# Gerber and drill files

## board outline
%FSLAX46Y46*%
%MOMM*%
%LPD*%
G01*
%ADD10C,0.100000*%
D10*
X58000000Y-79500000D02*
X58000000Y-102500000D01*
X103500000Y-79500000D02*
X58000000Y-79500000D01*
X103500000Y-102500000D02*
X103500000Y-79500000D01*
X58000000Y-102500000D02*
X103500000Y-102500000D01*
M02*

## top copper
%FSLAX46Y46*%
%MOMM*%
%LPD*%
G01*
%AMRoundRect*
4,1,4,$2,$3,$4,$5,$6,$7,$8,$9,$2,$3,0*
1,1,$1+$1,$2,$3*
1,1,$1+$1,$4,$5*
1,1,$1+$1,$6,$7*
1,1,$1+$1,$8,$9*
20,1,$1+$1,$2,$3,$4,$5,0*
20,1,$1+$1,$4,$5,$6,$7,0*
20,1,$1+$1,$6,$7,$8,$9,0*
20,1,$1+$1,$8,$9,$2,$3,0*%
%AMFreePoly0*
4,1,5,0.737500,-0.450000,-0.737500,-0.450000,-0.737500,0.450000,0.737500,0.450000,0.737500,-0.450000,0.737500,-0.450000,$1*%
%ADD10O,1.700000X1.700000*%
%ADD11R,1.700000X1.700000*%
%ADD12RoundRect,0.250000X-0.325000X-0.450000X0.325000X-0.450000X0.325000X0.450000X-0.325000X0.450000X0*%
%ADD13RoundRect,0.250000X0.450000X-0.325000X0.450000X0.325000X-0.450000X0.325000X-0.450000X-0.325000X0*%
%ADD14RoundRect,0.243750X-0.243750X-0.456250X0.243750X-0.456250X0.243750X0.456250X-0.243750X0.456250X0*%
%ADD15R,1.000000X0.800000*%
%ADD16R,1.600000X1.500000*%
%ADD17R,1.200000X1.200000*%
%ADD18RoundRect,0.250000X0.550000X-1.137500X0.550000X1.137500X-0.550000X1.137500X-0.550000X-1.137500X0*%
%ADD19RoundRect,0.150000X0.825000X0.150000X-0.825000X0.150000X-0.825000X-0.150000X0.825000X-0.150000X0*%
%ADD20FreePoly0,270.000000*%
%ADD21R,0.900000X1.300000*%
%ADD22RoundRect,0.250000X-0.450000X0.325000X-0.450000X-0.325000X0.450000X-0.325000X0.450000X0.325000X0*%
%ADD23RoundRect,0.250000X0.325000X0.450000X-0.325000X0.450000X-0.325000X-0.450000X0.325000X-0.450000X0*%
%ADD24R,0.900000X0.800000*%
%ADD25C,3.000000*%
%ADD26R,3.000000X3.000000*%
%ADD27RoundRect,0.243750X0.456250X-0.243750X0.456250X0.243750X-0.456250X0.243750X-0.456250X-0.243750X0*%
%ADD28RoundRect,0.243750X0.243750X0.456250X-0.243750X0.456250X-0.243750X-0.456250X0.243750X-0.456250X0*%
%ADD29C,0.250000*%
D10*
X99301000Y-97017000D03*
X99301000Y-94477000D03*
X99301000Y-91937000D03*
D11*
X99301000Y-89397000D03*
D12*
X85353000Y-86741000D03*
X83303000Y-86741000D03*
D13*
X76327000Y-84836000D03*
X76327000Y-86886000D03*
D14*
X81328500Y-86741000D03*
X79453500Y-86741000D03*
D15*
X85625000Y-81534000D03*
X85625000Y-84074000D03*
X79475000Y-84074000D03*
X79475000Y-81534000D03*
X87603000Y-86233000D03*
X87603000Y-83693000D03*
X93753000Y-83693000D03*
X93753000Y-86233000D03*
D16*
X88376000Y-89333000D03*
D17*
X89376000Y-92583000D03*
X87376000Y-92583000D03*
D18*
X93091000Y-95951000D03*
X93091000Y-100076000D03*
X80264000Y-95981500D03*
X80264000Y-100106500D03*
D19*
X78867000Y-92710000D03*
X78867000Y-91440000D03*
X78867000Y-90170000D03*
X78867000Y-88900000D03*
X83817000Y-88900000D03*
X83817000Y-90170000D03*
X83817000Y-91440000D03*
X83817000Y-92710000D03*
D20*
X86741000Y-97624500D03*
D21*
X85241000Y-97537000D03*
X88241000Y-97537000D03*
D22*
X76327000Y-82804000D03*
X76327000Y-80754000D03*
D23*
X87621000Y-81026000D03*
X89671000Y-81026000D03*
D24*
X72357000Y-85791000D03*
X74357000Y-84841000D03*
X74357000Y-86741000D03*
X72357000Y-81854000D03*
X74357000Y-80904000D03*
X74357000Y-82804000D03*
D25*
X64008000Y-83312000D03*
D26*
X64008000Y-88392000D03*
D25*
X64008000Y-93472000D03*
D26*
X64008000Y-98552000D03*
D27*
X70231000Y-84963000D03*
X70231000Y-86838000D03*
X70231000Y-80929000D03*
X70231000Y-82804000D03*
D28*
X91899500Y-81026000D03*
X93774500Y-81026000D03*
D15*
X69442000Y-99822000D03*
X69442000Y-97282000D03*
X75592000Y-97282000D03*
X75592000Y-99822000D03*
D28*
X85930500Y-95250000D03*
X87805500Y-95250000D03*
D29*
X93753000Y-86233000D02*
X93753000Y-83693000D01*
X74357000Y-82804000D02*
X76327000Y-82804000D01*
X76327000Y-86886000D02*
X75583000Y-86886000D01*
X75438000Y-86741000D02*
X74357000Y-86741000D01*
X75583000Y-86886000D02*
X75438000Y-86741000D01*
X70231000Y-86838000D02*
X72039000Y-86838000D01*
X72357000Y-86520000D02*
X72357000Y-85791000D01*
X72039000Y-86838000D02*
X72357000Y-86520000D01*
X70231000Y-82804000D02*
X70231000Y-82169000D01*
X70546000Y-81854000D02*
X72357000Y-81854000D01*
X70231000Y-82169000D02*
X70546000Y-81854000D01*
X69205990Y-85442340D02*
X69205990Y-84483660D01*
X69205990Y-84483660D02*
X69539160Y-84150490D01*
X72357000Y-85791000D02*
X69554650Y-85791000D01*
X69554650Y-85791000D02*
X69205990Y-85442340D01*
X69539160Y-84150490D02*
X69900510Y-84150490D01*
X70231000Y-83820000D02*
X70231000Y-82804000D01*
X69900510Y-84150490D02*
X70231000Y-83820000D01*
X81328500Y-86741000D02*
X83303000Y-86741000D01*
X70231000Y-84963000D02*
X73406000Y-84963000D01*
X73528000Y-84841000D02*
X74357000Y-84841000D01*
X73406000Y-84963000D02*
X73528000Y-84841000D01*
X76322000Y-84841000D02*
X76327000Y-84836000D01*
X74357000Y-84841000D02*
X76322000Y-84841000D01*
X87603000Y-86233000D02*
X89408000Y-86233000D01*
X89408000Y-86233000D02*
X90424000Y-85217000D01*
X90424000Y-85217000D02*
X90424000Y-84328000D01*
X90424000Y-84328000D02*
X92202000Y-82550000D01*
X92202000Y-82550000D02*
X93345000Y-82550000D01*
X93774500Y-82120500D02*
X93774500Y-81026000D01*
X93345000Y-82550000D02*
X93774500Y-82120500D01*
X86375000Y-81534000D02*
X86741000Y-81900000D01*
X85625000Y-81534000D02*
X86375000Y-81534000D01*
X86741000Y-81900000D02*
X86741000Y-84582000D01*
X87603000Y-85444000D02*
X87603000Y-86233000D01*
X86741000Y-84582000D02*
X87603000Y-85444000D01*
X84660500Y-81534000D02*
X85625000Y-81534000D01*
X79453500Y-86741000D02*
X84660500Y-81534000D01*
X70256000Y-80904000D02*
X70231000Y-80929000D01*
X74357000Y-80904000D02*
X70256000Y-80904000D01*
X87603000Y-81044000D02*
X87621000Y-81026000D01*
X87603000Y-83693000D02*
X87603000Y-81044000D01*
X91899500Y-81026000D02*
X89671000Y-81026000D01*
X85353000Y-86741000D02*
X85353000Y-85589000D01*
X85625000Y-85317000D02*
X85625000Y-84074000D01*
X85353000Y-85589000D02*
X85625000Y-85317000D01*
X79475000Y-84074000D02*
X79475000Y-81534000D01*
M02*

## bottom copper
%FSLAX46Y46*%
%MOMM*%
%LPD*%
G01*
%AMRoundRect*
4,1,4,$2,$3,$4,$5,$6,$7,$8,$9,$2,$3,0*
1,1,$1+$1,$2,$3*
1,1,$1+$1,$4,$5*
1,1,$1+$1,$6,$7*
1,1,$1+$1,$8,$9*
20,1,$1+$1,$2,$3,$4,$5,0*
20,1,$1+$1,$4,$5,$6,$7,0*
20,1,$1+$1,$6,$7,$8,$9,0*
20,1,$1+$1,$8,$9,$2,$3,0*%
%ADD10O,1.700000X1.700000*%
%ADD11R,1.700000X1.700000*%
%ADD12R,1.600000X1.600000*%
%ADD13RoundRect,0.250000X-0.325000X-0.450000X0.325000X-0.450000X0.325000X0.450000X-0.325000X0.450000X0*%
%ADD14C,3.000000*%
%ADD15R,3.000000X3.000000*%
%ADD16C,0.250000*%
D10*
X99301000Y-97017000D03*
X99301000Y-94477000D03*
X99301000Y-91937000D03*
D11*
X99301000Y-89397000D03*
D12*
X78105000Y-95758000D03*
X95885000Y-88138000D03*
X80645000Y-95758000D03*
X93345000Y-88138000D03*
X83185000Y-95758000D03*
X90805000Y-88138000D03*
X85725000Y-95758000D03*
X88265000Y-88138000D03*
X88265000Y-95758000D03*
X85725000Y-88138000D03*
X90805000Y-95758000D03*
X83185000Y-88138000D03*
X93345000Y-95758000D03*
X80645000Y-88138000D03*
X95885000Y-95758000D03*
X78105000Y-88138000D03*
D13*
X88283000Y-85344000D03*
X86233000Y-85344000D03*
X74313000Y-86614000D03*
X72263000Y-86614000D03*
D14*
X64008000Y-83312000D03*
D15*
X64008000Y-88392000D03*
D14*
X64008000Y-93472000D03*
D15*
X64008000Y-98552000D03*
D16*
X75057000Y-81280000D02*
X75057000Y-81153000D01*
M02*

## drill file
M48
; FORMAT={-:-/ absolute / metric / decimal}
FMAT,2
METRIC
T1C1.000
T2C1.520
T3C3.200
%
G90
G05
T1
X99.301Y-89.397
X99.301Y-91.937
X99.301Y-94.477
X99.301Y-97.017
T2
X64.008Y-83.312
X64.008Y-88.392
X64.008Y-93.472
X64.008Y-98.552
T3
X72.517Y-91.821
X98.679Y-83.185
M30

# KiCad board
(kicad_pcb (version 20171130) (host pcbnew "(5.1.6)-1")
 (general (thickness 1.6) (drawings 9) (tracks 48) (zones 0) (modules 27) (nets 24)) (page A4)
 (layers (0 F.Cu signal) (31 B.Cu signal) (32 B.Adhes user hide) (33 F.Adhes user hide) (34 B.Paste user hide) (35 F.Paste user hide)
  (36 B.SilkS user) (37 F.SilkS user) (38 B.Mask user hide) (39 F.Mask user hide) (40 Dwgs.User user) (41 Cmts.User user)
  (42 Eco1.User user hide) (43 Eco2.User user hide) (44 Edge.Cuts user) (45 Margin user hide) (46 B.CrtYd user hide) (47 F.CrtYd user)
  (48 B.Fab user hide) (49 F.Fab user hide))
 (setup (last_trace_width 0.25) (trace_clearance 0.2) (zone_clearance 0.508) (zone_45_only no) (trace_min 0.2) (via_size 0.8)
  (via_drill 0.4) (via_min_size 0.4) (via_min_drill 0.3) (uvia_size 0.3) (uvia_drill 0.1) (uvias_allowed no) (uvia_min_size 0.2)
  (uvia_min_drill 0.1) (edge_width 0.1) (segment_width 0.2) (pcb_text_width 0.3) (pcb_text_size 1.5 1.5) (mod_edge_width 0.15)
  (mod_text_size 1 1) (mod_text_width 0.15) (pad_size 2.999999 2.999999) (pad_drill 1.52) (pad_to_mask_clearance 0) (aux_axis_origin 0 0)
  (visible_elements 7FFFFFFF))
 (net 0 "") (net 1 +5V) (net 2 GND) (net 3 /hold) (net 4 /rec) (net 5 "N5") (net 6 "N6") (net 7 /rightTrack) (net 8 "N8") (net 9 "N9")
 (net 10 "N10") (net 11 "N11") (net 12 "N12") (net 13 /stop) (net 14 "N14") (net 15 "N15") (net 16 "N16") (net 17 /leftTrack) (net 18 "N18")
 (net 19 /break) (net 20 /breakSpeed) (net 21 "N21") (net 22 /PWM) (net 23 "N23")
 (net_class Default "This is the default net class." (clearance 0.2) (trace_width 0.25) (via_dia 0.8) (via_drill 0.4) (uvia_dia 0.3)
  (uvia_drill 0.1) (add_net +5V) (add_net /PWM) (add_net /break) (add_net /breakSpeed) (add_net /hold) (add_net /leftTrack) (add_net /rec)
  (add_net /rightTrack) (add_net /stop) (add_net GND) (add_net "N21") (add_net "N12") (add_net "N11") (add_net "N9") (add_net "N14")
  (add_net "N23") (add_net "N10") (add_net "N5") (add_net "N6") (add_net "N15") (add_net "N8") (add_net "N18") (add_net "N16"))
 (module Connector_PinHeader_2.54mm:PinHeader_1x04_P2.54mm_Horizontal (layer F.Cu) (at 99.301 89.397)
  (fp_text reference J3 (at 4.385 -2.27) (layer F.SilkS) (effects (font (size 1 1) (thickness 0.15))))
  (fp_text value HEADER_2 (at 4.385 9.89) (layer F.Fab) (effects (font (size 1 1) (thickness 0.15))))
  (pad 4 thru_hole oval (at 0 7.62) (size 1.7 1.7) (drill 1) (layers *.Cu *.Mask) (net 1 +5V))
  (pad 3 thru_hole oval (at 0 5.08) (size 1.7 1.7) (drill 1) (layers *.Cu *.Mask) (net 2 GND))
  (pad 2 thru_hole oval (at 0 2.54) (size 1.7 1.7) (drill 1) (layers *.Cu *.Mask) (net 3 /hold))
  (pad 1 thru_hole rect (at 0 0) (size 1.7 1.7) (drill 1) (layers *.Cu *.Mask) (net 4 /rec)))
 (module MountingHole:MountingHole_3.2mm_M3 (layer F.Cu) (at 98.679 83.185)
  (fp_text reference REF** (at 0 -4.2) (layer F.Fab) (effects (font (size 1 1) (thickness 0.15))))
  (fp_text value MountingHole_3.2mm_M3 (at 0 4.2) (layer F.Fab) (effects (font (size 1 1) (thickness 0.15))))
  (pad 1 np_thru_hole circle (at 0 0) (size 3.2 3.2) (drill 3.2) (layers *.Cu *.Mask)))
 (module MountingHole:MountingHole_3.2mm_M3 (layer F.Cu) (at 72.517 91.821)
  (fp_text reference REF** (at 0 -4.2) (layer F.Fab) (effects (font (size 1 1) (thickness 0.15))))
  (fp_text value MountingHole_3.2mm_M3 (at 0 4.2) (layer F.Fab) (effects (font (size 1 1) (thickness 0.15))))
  (pad 1 np_thru_hole circle (at 0 0) (size 3.2 3.2) (drill 3.2) (layers *.Cu *.Mask)))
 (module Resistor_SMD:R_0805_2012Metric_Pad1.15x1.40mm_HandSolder (layer F.Cu) (at 84.328 86.741)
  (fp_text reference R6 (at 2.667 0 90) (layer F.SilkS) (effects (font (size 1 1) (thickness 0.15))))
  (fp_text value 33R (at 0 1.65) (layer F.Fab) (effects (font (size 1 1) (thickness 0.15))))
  (pad 2 smd roundrect (at 1.025 0) (size 1.15 1.4) (layers F.Cu F.Paste F.Mask) (roundrect_rratio 0.217391) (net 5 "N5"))
  (pad 1 smd roundrect (at -1.025 0) (size 1.15 1.4) (layers F.Cu F.Paste F.Mask) (roundrect_rratio 0.217391) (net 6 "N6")))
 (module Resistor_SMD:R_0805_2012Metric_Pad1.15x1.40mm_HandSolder (layer F.Cu) (at 76.327 85.861 90)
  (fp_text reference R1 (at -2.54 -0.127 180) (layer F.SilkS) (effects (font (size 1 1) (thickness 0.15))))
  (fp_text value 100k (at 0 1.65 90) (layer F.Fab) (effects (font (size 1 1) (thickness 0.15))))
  (pad 2 smd roundrect (at 1.025 0 90) (size 1.15 1.4) (layers F.Cu F.Paste F.Mask) (roundrect_rratio 0.217391) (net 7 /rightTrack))
  (pad 1 smd roundrect (at -1.025 0 90) (size 1.15 1.4) (layers F.Cu F.Paste F.Mask) (roundrect_rratio 0.217391) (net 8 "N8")))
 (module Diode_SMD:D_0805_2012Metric (layer F.Cu) (at 80.391 86.741)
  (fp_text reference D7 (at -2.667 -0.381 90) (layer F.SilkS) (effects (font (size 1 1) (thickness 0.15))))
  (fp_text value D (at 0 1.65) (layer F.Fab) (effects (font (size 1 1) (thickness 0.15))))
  (pad 2 smd roundrect (at 0.9375 0) (size 0.975 1.4) (layers F.Cu F.Paste F.Mask) (roundrect_rratio 0.25) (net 6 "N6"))
  (pad 1 smd roundrect (at -0.9375 0) (size 0.975 1.4) (layers F.Cu F.Paste F.Mask) (roundrect_rratio 0.25) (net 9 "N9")))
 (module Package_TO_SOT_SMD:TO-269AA (layer F.Cu) (at 82.55 82.804)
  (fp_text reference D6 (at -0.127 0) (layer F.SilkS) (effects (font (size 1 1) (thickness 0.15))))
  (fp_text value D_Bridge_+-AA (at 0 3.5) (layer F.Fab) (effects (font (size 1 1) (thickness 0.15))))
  (pad 4 smd rect (at 3.075 -1.27) (size 1 0.8) (layers F.Cu F.Paste F.Mask) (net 9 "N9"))
  (pad 3 smd rect (at 3.075 1.27) (size 1 0.8) (layers F.Cu F.Paste F.Mask) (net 5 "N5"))
  (pad 2 smd rect (at -3.075 1.27) (size 1 0.8) (layers F.Cu F.Paste F.Mask) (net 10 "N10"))
  (pad 1 smd rect (at -3.075 -1.27) (size 1 0.8) (layers F.Cu F.Paste F.Mask) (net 10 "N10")))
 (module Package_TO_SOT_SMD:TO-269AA (layer F.Cu) (at 90.678 84.963 180)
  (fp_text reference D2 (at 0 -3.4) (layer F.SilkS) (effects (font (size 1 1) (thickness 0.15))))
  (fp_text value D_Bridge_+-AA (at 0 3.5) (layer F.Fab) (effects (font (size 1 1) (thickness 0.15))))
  (pad 4 smd rect (at 3.075 -1.27 180) (size 1 0.8) (layers F.Cu F.Paste F.Mask) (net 9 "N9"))
  (pad 3 smd rect (at 3.075 1.27 180) (size 1 0.8) (layers F.Cu F.Paste F.Mask) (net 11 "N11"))
  (pad 2 smd rect (at -3.075 1.27 180) (size 1 0.8) (layers F.Cu F.Paste F.Mask) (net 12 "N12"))
  (pad 1 smd rect (at -3.075 -1.27 180) (size 1 0.8) (layers F.Cu F.Paste F.Mask) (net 12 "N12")))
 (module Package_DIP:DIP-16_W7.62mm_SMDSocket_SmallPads (layer B.Cu) (at 86.995 91.948 270)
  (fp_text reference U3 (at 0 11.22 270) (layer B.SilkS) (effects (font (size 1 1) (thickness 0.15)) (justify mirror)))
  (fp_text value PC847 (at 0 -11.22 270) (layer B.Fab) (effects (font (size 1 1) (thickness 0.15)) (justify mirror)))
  (pad 16 smd rect (at 3.81 8.89 270) (size 1.6 1.6) (layers B.Cu B.Paste B.Mask) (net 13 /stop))
  (pad 8 smd rect (at -3.81 -8.89 270) (size 1.6 1.6) (layers B.Cu B.Paste B.Mask) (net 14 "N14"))
  (pad 15 smd rect (at 3.81 6.35 270) (size 1.6 1.6) (layers B.Cu B.Paste B.Mask) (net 2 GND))
  (pad 7 smd rect (at -3.81 -6.35 270) (size 1.6 1.6) (layers B.Cu B.Paste B.Mask) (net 9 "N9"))
  (pad 14 smd rect (at 3.81 3.81 270) (size 1.6 1.6) (layers B.Cu B.Paste B.Mask) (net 7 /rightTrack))
  (pad 6 smd rect (at -3.81 -3.81 270) (size 1.6 1.6) (layers B.Cu B.Paste B.Mask) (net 2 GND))
  (pad 13 smd rect (at 3.81 1.27 270) (size 1.6 1.6) (layers B.Cu B.Paste B.Mask) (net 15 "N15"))
  (pad 5 smd rect (at -3.81 -1.27 270) (size 1.6 1.6) (layers B.Cu B.Paste B.Mask) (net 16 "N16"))
  (pad 12 smd rect (at 3.81 -1.27 270) (size 1.6 1.6) (layers B.Cu B.Paste B.Mask) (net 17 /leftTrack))
  (pad 4 smd rect (at -3.81 1.27 270) (size 1.6 1.6) (layers B.Cu B.Paste B.Mask) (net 2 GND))
  (pad 11 smd rect (at 3.81 -3.81 270) (size 1.6 1.6) (layers B.Cu B.Paste B.Mask) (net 8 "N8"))
  (pad 3 smd rect (at -3.81 3.81 270) (size 1.6 1.6) (layers B.Cu B.Paste B.Mask) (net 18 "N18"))
  (pad 10 smd rect (at 3.81 -6.35 270) (size 1.6 1.6) (layers B.Cu B.Paste B.Mask) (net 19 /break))
  (pad 2 smd rect (at -3.81 6.35 270) (size 1.6 1.6) (layers B.Cu B.Paste B.Mask) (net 6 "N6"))
  (pad 9 smd rect (at 3.81 -8.89 270) (size 1.6 1.6) (layers B.Cu B.Paste B.Mask) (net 2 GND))
  (pad 1 smd rect (at -3.81 8.89 270) (size 1.6 1.6) (layers B.Cu B.Paste B.Mask) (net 9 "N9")))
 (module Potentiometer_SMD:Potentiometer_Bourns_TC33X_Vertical (layer F.Cu) (at 88.376 90.783 90)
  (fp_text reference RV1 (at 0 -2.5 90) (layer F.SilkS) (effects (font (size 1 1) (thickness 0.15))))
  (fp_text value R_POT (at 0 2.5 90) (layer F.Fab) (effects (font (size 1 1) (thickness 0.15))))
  (pad 2 smd rect (at 1.45 0 90) (size 1.5 1.6) (layers F.Cu F.Paste F.Mask) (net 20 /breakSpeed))
  (pad 3 smd rect (at -1.8 1 90) (size 1.2 1.2) (layers F.Cu F.Paste F.Mask) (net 1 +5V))
  (pad 1 smd rect (at -1.8 -1 90) (size 1.2 1.2) (layers F.Cu F.Paste F.Mask) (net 2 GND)))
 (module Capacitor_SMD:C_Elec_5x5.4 (layer F.Cu) (at 93.091 98.0135 90)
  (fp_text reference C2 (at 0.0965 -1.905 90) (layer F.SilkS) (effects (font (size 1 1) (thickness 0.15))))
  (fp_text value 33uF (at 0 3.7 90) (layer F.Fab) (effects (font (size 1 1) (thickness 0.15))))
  (pad 2 smd roundrect (at 2.0625 0 90) (size 2.775 1.6) (layers F.Cu F.Paste F.Mask) (roundrect_rratio 0.15625) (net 2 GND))
  (pad 1 smd roundrect (at -2.0625 0 90) (size 2.775 1.6) (layers F.Cu F.Paste F.Mask) (roundrect_rratio 0.15625) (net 1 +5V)))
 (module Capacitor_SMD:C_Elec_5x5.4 (layer F.Cu) (at 80.264 98.044 90)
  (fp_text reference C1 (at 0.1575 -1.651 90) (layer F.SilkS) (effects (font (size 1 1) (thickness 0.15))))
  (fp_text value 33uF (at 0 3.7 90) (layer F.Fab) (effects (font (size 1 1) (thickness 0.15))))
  (pad 2 smd roundrect (at 2.0625 0 90) (size 2.775 1.6) (layers F.Cu F.Paste F.Mask) (roundrect_rratio 0.15625) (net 2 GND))
  (pad 1 smd roundrect (at -2.0625 0 90) (size 2.775 1.6) (layers F.Cu F.Paste F.Mask) (roundrect_rratio 0.15625) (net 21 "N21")))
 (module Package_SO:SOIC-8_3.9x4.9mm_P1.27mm (layer F.Cu) (at 81.342 90.805 180)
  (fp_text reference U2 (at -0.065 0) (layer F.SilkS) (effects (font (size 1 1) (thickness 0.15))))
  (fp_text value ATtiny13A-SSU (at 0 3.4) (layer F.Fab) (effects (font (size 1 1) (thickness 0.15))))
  (pad 8 smd roundrect (at 2.475 -1.905 180) (size 1.95 0.6) (layers F.Cu F.Paste F.Mask) (roundrect_rratio 0.25) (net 1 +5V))
  (pad 7 smd roundrect (at 2.475 -0.635 180) (size 1.95 0.6) (layers F.Cu F.Paste F.Mask) (roundrect_rratio 0.25) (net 19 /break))
  (pad 6 smd roundrect (at 2.475 0.635 180) (size 1.95 0.6) (layers F.Cu F.Paste F.Mask) (roundrect_rratio 0.25) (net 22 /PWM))
  (pad 5 smd roundrect (at 2.475 1.905 180) (size 1.95 0.6) (layers F.Cu F.Paste F.Mask) (roundrect_rratio 0.25) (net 4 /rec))
  (pad 4 smd roundrect (at -2.475 1.905 180) (size 1.95 0.6) (layers F.Cu F.Paste F.Mask) (roundrect_rratio 0.25) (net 2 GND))
  (pad 3 smd roundrect (at -2.475 0.635 180) (size 1.95 0.6) (layers F.Cu F.Paste F.Mask) (roundrect_rratio 0.25) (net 20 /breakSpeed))
  (pad 2 smd roundrect (at -2.475 -0.635 180) (size 1.95 0.6) (layers F.Cu F.Paste F.Mask) (roundrect_rratio 0.25) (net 3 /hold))
  (pad 1 smd roundrect (at -2.475 -1.905 180) (size 1.95 0.6) (layers F.Cu F.Paste F.Mask) (roundrect_rratio 0.25) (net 13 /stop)))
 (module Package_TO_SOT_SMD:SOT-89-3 (layer F.Cu) (at 86.741 99.187 270)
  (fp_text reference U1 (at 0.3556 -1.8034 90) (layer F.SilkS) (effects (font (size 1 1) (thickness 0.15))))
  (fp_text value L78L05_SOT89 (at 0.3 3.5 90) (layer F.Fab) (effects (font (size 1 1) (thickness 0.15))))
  (pad 2 smd custom (at -1.5625 0 270) (size 1.475 0.9) (layers F.Cu F.Paste F.Mask) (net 2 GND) (zone_connect 2)
   (options (clearance outline) (anchor rect)) (primitives))
  (pad 3 smd rect (at -1.65 1.5 270) (size 1.3 0.9) (layers F.Cu F.Paste F.Mask) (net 21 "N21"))
  (pad 1 smd rect (at -1.65 -1.5 270) (size 1.3 0.9) (layers F.Cu F.Paste F.Mask) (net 1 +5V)))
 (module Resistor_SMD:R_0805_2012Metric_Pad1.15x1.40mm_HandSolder (layer F.Cu) (at 76.327 81.779 270)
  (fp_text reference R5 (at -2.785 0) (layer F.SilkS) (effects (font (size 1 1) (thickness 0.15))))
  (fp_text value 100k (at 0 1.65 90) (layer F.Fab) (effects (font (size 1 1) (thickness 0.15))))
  (pad 2 smd roundrect (at 1.025 0 270) (size 1.15 1.4) (layers F.Cu F.Paste F.Mask) (roundrect_rratio 0.217391) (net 15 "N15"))
  (pad 1 smd roundrect (at -1.025 0 270) (size 1.15 1.4) (layers F.Cu F.Paste F.Mask) (roundrect_rratio 0.217391) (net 17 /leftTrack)))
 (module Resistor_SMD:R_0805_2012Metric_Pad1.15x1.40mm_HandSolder (layer F.Cu) (at 88.646 81.026 180)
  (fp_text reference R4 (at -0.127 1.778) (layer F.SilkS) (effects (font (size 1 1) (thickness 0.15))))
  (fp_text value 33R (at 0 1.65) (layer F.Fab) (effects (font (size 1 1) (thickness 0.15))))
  (pad 2 smd roundrect (at 1.025 0 180) (size 1.15 1.4) (layers F.Cu F.Paste F.Mask) (roundrect_rratio 0.217391) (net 11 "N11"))
  (pad 1 smd roundrect (at -1.025 0 180) (size 1.15 1.4) (layers F.Cu F.Paste F.Mask) (roundrect_rratio 0.217391) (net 14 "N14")))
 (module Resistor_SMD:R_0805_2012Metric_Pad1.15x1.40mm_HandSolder (layer B.Cu) (at 87.258 85.344)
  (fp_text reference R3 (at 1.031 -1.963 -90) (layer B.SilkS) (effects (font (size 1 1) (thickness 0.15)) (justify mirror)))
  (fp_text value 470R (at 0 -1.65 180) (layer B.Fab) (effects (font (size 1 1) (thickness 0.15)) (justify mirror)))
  (pad 2 smd roundrect (at 1.025 0) (size 1.15 1.4) (layers B.Cu B.Paste B.Mask) (roundrect_rratio 0.217391) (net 16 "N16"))
  (pad 1 smd roundrect (at -1.025 0) (size 1.15 1.4) (layers B.Cu B.Paste B.Mask) (roundrect_rratio 0.217391) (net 22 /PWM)))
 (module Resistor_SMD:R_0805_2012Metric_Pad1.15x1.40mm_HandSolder (layer B.Cu) (at 73.288 86.614)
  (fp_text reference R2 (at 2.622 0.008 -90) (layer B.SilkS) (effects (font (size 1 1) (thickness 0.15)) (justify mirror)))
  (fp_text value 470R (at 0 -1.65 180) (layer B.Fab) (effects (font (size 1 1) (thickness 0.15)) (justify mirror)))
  (pad 2 smd roundrect (at 1.025 0) (size 1.15 1.4) (layers B.Cu B.Paste B.Mask) (roundrect_rratio 0.217391) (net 18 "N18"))
  (pad 1 smd roundrect (at -1.025 0) (size 1.15 1.4) (layers B.Cu B.Paste B.Mask) (roundrect_rratio 0.217391) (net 22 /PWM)))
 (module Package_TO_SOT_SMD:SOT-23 (layer F.Cu) (at 73.357 85.791 180)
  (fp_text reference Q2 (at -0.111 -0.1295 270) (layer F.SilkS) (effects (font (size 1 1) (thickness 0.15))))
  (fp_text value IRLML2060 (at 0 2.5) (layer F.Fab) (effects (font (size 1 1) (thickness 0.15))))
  (pad 3 smd rect (at 1 0 180) (size 0.9 0.8) (layers F.Cu F.Paste F.Mask) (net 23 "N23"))
  (pad 2 smd rect (at -1 0.95 180) (size 0.9 0.8) (layers F.Cu F.Paste F.Mask) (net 7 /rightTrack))
  (pad 1 smd rect (at -1 -0.95 180) (size 0.9 0.8) (layers F.Cu F.Paste F.Mask) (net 8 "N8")))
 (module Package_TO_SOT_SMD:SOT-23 (layer F.Cu) (at 73.357 81.854 180)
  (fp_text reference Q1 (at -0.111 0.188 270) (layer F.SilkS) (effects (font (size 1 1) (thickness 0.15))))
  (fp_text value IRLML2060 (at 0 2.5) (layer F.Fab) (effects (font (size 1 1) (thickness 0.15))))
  (pad 3 smd rect (at 1 0 180) (size 0.9 0.8) (layers F.Cu F.Paste F.Mask) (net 23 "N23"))
  (pad 2 smd rect (at -1 0.95 180) (size 0.9 0.8) (layers F.Cu F.Paste F.Mask) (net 9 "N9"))
  (pad 1 smd rect (at -1 -0.95 180) (size 0.9 0.8) (layers F.Cu F.Paste F.Mask) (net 15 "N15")))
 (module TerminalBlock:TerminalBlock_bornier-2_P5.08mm (layer F.Cu) (at 64.008 88.392 90)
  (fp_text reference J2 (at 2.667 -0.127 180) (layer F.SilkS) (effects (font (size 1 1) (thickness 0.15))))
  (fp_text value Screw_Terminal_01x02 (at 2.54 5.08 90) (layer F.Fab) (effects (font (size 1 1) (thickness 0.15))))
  (pad 2 thru_hole circle (at 5.08 0 90) (size 3 3) (drill 1.52) (layers *.Cu *.Mask) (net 5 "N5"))
  (pad 1 thru_hole rect (at 0 0 90) (size 3 3) (drill 1.52) (layers *.Cu *.Mask) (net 11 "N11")))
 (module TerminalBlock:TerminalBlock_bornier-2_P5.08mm (layer F.Cu) (at 64.008 98.552 90)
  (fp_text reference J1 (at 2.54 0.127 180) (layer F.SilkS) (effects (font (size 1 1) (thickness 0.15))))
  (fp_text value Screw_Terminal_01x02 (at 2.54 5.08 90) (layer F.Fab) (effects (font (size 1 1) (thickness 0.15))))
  (pad 2 thru_hole circle (at 5.08 0 90) (size 3 3) (drill 1.52) (layers *.Cu *.Mask) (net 17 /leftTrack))
  (pad 1 thru_hole rect (at 0 0 90) (size 3 3) (drill 1.52) (layers *.Cu *.Mask) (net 7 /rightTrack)))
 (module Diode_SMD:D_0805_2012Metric (layer F.Cu) (at 70.231 85.9005 90)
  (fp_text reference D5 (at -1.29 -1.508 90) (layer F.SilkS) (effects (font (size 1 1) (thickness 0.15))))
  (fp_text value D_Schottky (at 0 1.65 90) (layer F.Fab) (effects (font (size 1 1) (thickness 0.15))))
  (pad 2 smd roundrect (at 0.9375 0 90) (size 0.975 1.4) (layers F.Cu F.Paste F.Mask) (roundrect_rratio 0.25) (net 7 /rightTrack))
  (pad 1 smd roundrect (at -0.9375 0 90) (size 0.975 1.4) (layers F.Cu F.Paste F.Mask) (roundrect_rratio 0.25) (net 23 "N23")))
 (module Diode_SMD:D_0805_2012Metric (layer F.Cu) (at 70.231 81.8665 90)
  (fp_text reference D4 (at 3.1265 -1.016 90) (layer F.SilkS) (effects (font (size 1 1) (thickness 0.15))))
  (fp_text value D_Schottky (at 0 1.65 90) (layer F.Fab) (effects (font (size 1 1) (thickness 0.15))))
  (pad 2 smd roundrect (at 0.9375 0 90) (size 0.975 1.4) (layers F.Cu F.Paste F.Mask) (roundrect_rratio 0.25) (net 9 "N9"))
  (pad 1 smd roundrect (at -0.9375 0 90) (size 0.975 1.4) (layers F.Cu F.Paste F.Mask) (roundrect_rratio 0.25) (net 23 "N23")))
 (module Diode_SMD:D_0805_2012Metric (layer F.Cu) (at 92.837 81.026 180)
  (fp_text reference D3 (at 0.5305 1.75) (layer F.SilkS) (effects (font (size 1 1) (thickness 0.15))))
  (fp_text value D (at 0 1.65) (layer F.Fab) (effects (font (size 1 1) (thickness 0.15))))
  (pad 2 smd roundrect (at 0.9375 0 180) (size 0.975 1.4) (layers F.Cu F.Paste F.Mask) (roundrect_rratio 0.25) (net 14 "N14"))
  (pad 1 smd roundrect (at -0.9375 0 180) (size 0.975 1.4) (layers F.Cu F.Paste F.Mask) (roundrect_rratio 0.25) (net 9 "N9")))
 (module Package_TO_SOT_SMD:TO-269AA (layer F.Cu) (at 72.517 98.552 180)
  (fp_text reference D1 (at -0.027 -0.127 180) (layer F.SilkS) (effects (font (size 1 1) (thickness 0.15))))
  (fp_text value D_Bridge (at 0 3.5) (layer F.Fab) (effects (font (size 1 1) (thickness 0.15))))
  (pad 4 smd rect (at 3.075 -1.27 180) (size 1 0.8) (layers F.Cu F.Paste F.Mask) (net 7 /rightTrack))
  (pad 3 smd rect (at 3.075 1.27 180) (size 1 0.8) (layers F.Cu F.Paste F.Mask) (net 17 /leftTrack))
  (pad 2 smd rect (at -3.075 1.27 180) (size 1 0.8) (layers F.Cu F.Paste F.Mask) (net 2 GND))
  (pad 1 smd rect (at -3.075 -1.27 180) (size 1 0.8) (layers F.Cu F.Paste F.Mask) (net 21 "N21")))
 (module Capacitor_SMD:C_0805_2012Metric (layer F.Cu) (at 86.868 95.25 180)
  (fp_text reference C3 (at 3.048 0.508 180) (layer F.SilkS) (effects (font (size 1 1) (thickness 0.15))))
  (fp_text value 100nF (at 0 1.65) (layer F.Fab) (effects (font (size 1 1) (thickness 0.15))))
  (pad 2 smd roundrect (at 0.9375 0 180) (size 0.975 1.4) (layers F.Cu F.Paste F.Mask) (roundrect_rratio 0.25) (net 1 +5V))
  (pad 1 smd roundrect (at -0.9375 0 180) (size 0.975 1.4) (layers F.Cu F.Paste F.Mask) (roundrect_rratio 0.25) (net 2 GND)))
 (gr_line (start 58 79.5) (end 58 102.5) (layer Edge.Cuts) (width 0.1))
 (gr_line (start 103.5 79.5) (end 58 79.5) (layer Edge.Cuts) (width 0.1))
 (gr_line (start 103.5 102.5) (end 103.5 79.5) (layer Edge.Cuts) (width 0.1))
 (gr_line (start 58 102.5) (end 103.5 102.5) (layer Edge.Cuts) (width 0.1))
 (segment (start 75.057 81.28) (end 75.057 81.153) (width 0.25) (layer B.Cu) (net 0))
 (segment (start 93.753 86.233) (end 93.753 83.693) (width 0.25) (layer F.Cu) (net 12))
 (segment (start 74.357 82.804) (end 76.327 82.804) (width 0.25) (layer F.Cu) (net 15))
 (segment (start 76.327 86.886) (end 75.583 86.886) (width 0.25) (layer F.Cu) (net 8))
 (segment (start 75.438 86.741) (end 74.357 86.741) (width 0.25) (layer F.Cu) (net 8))
 (segment (start 75.583 86.886) (end 75.438 86.741) (width 0.25) (layer F.Cu) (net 8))
 (segment (start 70.231 86.838) (end 72.039 86.838) (width 0.25) (layer F.Cu) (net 23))
 (segment (start 72.357 86.52) (end 72.357 85.791) (width 0.25) (layer F.Cu) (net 23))
 (segment (start 72.039 86.838) (end 72.357 86.52) (width 0.25) (layer F.Cu) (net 23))
 (segment (start 70.231 82.804) (end 70.231 82.169) (width 0.25) (layer F.Cu) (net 23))
 (segment (start 70.546 81.854) (end 72.357 81.854) (width 0.25) (layer F.Cu) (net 23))
 (segment (start 70.231 82.169) (end 70.546 81.854) (width 0.25) (layer F.Cu) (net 23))
 (segment (start 69.20599 85.44234) (end 69.20599 84.48366) (width 0.25) (layer F.Cu) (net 23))
 (segment (start 69.20599 84.48366) (end 69.53916 84.15049) (width 0.25) (layer F.Cu) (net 23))
 (segment (start 72.357 85.791) (end 69.55465 85.791) (width 0.25) (layer F.Cu) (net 23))
 (segment (start 69.55465 85.791) (end 69.20599 85.44234) (width 0.25) (layer F.Cu) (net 23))
 (segment (start 69.53916 84.15049) (end 69.90051 84.15049) (width 0.25) (layer F.Cu) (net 23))
 (segment (start 70.231 83.82) (end 70.231 82.804) (width 0.25) (layer F.Cu) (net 23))
 (segment (start 69.90051 84.15049) (end 70.231 83.82) (width 0.25) (layer F.Cu) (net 23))
 (segment (start 81.3285 86.741) (end 83.303 86.741) (width 0.25) (layer F.Cu) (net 6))
 (segment (start 70.231 84.963) (end 73.406 84.963) (width 0.25) (layer F.Cu) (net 7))
 (segment (start 73.528 84.841) (end 74.357 84.841) (width 0.25) (layer F.Cu) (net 7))
 (segment (start 73.406 84.963) (end 73.528 84.841) (width 0.25) (layer F.Cu) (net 7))
 (segment (start 76.322 84.841) (end 76.327 84.836) (width 0.25) (layer F.Cu) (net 7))
 (segment (start 74.357 84.841) (end 76.322 84.841) (width 0.25) (layer F.Cu) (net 7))
 (segment (start 87.603 86.233) (end 89.408 86.233) (width 0.25) (layer F.Cu) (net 9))
 (segment (start 89.408 86.233) (end 90.424 85.217) (width 0.25) (layer F.Cu) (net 9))
 (segment (start 90.424 85.217) (end 90.424 84.328) (width 0.25) (layer F.Cu) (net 9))
 (segment (start 90.424 84.328) (end 92.202 82.55) (width 0.25) (layer F.Cu) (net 9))
 (segment (start 92.202 82.55) (end 93.345 82.55) (width 0.25) (layer F.Cu) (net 9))
 (segment (start 93.7745 82.1205) (end 93.7745 81.026) (width 0.25) (layer F.Cu) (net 9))
 (segment (start 93.345 82.55) (end 93.7745 82.1205) (width 0.25) (layer F.Cu) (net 9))
 (segment (start 86.375 81.534) (end 86.741 81.9) (width 0.25) (layer F.Cu) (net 9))
 (segment (start 85.625 81.534) (end 86.375 81.534) (width 0.25) (layer F.Cu) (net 9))
 (segment (start 86.741 81.9) (end 86.741 84.582) (width 0.25) (layer F.Cu) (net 9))
 (segment (start 87.603 85.444) (end 87.603 86.233) (width 0.25) (layer F.Cu) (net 9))
 (segment (start 86.741 84.582) (end 87.603 85.444) (width 0.25) (layer F.Cu) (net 9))
 (segment (start 84.6605 81.534) (end 85.625 81.534) (width 0.25) (layer F.Cu) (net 9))
 (segment (start 79.4535 86.741) (end 84.6605 81.534) (width 0.25) (layer F.Cu) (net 9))
 (segment (start 70.256 80.904) (end 70.231 80.929) (width 0.25) (layer F.Cu) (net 9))
 (segment (start 74.357 80.904) (end 70.256 80.904) (width 0.25) (layer F.Cu) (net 9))
 (segment (start 87.603 81.044) (end 87.621 81.026) (width 0.25) (layer F.Cu) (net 11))
 (segment (start 87.603 83.693) (end 87.603 81.044) (width 0.25) (layer F.Cu) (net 11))
 (segment (start 91.8995 81.026) (end 89.671 81.026) (width 0.25) (layer F.Cu) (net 14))
 (segment (start 85.353 86.741) (end 85.353 85.589) (width 0.25) (layer F.Cu) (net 5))
 (segment (start 85.625 85.317) (end 85.625 84.074) (width 0.25) (layer F.Cu) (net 5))
 (segment (start 85.353 85.589) (end 85.625 85.317) (width 0.25) (layer F.Cu) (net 5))
 (segment (start 79.475 84.074) (end 79.475 81.534) (width 0.25) (layer F.Cu) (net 10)))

